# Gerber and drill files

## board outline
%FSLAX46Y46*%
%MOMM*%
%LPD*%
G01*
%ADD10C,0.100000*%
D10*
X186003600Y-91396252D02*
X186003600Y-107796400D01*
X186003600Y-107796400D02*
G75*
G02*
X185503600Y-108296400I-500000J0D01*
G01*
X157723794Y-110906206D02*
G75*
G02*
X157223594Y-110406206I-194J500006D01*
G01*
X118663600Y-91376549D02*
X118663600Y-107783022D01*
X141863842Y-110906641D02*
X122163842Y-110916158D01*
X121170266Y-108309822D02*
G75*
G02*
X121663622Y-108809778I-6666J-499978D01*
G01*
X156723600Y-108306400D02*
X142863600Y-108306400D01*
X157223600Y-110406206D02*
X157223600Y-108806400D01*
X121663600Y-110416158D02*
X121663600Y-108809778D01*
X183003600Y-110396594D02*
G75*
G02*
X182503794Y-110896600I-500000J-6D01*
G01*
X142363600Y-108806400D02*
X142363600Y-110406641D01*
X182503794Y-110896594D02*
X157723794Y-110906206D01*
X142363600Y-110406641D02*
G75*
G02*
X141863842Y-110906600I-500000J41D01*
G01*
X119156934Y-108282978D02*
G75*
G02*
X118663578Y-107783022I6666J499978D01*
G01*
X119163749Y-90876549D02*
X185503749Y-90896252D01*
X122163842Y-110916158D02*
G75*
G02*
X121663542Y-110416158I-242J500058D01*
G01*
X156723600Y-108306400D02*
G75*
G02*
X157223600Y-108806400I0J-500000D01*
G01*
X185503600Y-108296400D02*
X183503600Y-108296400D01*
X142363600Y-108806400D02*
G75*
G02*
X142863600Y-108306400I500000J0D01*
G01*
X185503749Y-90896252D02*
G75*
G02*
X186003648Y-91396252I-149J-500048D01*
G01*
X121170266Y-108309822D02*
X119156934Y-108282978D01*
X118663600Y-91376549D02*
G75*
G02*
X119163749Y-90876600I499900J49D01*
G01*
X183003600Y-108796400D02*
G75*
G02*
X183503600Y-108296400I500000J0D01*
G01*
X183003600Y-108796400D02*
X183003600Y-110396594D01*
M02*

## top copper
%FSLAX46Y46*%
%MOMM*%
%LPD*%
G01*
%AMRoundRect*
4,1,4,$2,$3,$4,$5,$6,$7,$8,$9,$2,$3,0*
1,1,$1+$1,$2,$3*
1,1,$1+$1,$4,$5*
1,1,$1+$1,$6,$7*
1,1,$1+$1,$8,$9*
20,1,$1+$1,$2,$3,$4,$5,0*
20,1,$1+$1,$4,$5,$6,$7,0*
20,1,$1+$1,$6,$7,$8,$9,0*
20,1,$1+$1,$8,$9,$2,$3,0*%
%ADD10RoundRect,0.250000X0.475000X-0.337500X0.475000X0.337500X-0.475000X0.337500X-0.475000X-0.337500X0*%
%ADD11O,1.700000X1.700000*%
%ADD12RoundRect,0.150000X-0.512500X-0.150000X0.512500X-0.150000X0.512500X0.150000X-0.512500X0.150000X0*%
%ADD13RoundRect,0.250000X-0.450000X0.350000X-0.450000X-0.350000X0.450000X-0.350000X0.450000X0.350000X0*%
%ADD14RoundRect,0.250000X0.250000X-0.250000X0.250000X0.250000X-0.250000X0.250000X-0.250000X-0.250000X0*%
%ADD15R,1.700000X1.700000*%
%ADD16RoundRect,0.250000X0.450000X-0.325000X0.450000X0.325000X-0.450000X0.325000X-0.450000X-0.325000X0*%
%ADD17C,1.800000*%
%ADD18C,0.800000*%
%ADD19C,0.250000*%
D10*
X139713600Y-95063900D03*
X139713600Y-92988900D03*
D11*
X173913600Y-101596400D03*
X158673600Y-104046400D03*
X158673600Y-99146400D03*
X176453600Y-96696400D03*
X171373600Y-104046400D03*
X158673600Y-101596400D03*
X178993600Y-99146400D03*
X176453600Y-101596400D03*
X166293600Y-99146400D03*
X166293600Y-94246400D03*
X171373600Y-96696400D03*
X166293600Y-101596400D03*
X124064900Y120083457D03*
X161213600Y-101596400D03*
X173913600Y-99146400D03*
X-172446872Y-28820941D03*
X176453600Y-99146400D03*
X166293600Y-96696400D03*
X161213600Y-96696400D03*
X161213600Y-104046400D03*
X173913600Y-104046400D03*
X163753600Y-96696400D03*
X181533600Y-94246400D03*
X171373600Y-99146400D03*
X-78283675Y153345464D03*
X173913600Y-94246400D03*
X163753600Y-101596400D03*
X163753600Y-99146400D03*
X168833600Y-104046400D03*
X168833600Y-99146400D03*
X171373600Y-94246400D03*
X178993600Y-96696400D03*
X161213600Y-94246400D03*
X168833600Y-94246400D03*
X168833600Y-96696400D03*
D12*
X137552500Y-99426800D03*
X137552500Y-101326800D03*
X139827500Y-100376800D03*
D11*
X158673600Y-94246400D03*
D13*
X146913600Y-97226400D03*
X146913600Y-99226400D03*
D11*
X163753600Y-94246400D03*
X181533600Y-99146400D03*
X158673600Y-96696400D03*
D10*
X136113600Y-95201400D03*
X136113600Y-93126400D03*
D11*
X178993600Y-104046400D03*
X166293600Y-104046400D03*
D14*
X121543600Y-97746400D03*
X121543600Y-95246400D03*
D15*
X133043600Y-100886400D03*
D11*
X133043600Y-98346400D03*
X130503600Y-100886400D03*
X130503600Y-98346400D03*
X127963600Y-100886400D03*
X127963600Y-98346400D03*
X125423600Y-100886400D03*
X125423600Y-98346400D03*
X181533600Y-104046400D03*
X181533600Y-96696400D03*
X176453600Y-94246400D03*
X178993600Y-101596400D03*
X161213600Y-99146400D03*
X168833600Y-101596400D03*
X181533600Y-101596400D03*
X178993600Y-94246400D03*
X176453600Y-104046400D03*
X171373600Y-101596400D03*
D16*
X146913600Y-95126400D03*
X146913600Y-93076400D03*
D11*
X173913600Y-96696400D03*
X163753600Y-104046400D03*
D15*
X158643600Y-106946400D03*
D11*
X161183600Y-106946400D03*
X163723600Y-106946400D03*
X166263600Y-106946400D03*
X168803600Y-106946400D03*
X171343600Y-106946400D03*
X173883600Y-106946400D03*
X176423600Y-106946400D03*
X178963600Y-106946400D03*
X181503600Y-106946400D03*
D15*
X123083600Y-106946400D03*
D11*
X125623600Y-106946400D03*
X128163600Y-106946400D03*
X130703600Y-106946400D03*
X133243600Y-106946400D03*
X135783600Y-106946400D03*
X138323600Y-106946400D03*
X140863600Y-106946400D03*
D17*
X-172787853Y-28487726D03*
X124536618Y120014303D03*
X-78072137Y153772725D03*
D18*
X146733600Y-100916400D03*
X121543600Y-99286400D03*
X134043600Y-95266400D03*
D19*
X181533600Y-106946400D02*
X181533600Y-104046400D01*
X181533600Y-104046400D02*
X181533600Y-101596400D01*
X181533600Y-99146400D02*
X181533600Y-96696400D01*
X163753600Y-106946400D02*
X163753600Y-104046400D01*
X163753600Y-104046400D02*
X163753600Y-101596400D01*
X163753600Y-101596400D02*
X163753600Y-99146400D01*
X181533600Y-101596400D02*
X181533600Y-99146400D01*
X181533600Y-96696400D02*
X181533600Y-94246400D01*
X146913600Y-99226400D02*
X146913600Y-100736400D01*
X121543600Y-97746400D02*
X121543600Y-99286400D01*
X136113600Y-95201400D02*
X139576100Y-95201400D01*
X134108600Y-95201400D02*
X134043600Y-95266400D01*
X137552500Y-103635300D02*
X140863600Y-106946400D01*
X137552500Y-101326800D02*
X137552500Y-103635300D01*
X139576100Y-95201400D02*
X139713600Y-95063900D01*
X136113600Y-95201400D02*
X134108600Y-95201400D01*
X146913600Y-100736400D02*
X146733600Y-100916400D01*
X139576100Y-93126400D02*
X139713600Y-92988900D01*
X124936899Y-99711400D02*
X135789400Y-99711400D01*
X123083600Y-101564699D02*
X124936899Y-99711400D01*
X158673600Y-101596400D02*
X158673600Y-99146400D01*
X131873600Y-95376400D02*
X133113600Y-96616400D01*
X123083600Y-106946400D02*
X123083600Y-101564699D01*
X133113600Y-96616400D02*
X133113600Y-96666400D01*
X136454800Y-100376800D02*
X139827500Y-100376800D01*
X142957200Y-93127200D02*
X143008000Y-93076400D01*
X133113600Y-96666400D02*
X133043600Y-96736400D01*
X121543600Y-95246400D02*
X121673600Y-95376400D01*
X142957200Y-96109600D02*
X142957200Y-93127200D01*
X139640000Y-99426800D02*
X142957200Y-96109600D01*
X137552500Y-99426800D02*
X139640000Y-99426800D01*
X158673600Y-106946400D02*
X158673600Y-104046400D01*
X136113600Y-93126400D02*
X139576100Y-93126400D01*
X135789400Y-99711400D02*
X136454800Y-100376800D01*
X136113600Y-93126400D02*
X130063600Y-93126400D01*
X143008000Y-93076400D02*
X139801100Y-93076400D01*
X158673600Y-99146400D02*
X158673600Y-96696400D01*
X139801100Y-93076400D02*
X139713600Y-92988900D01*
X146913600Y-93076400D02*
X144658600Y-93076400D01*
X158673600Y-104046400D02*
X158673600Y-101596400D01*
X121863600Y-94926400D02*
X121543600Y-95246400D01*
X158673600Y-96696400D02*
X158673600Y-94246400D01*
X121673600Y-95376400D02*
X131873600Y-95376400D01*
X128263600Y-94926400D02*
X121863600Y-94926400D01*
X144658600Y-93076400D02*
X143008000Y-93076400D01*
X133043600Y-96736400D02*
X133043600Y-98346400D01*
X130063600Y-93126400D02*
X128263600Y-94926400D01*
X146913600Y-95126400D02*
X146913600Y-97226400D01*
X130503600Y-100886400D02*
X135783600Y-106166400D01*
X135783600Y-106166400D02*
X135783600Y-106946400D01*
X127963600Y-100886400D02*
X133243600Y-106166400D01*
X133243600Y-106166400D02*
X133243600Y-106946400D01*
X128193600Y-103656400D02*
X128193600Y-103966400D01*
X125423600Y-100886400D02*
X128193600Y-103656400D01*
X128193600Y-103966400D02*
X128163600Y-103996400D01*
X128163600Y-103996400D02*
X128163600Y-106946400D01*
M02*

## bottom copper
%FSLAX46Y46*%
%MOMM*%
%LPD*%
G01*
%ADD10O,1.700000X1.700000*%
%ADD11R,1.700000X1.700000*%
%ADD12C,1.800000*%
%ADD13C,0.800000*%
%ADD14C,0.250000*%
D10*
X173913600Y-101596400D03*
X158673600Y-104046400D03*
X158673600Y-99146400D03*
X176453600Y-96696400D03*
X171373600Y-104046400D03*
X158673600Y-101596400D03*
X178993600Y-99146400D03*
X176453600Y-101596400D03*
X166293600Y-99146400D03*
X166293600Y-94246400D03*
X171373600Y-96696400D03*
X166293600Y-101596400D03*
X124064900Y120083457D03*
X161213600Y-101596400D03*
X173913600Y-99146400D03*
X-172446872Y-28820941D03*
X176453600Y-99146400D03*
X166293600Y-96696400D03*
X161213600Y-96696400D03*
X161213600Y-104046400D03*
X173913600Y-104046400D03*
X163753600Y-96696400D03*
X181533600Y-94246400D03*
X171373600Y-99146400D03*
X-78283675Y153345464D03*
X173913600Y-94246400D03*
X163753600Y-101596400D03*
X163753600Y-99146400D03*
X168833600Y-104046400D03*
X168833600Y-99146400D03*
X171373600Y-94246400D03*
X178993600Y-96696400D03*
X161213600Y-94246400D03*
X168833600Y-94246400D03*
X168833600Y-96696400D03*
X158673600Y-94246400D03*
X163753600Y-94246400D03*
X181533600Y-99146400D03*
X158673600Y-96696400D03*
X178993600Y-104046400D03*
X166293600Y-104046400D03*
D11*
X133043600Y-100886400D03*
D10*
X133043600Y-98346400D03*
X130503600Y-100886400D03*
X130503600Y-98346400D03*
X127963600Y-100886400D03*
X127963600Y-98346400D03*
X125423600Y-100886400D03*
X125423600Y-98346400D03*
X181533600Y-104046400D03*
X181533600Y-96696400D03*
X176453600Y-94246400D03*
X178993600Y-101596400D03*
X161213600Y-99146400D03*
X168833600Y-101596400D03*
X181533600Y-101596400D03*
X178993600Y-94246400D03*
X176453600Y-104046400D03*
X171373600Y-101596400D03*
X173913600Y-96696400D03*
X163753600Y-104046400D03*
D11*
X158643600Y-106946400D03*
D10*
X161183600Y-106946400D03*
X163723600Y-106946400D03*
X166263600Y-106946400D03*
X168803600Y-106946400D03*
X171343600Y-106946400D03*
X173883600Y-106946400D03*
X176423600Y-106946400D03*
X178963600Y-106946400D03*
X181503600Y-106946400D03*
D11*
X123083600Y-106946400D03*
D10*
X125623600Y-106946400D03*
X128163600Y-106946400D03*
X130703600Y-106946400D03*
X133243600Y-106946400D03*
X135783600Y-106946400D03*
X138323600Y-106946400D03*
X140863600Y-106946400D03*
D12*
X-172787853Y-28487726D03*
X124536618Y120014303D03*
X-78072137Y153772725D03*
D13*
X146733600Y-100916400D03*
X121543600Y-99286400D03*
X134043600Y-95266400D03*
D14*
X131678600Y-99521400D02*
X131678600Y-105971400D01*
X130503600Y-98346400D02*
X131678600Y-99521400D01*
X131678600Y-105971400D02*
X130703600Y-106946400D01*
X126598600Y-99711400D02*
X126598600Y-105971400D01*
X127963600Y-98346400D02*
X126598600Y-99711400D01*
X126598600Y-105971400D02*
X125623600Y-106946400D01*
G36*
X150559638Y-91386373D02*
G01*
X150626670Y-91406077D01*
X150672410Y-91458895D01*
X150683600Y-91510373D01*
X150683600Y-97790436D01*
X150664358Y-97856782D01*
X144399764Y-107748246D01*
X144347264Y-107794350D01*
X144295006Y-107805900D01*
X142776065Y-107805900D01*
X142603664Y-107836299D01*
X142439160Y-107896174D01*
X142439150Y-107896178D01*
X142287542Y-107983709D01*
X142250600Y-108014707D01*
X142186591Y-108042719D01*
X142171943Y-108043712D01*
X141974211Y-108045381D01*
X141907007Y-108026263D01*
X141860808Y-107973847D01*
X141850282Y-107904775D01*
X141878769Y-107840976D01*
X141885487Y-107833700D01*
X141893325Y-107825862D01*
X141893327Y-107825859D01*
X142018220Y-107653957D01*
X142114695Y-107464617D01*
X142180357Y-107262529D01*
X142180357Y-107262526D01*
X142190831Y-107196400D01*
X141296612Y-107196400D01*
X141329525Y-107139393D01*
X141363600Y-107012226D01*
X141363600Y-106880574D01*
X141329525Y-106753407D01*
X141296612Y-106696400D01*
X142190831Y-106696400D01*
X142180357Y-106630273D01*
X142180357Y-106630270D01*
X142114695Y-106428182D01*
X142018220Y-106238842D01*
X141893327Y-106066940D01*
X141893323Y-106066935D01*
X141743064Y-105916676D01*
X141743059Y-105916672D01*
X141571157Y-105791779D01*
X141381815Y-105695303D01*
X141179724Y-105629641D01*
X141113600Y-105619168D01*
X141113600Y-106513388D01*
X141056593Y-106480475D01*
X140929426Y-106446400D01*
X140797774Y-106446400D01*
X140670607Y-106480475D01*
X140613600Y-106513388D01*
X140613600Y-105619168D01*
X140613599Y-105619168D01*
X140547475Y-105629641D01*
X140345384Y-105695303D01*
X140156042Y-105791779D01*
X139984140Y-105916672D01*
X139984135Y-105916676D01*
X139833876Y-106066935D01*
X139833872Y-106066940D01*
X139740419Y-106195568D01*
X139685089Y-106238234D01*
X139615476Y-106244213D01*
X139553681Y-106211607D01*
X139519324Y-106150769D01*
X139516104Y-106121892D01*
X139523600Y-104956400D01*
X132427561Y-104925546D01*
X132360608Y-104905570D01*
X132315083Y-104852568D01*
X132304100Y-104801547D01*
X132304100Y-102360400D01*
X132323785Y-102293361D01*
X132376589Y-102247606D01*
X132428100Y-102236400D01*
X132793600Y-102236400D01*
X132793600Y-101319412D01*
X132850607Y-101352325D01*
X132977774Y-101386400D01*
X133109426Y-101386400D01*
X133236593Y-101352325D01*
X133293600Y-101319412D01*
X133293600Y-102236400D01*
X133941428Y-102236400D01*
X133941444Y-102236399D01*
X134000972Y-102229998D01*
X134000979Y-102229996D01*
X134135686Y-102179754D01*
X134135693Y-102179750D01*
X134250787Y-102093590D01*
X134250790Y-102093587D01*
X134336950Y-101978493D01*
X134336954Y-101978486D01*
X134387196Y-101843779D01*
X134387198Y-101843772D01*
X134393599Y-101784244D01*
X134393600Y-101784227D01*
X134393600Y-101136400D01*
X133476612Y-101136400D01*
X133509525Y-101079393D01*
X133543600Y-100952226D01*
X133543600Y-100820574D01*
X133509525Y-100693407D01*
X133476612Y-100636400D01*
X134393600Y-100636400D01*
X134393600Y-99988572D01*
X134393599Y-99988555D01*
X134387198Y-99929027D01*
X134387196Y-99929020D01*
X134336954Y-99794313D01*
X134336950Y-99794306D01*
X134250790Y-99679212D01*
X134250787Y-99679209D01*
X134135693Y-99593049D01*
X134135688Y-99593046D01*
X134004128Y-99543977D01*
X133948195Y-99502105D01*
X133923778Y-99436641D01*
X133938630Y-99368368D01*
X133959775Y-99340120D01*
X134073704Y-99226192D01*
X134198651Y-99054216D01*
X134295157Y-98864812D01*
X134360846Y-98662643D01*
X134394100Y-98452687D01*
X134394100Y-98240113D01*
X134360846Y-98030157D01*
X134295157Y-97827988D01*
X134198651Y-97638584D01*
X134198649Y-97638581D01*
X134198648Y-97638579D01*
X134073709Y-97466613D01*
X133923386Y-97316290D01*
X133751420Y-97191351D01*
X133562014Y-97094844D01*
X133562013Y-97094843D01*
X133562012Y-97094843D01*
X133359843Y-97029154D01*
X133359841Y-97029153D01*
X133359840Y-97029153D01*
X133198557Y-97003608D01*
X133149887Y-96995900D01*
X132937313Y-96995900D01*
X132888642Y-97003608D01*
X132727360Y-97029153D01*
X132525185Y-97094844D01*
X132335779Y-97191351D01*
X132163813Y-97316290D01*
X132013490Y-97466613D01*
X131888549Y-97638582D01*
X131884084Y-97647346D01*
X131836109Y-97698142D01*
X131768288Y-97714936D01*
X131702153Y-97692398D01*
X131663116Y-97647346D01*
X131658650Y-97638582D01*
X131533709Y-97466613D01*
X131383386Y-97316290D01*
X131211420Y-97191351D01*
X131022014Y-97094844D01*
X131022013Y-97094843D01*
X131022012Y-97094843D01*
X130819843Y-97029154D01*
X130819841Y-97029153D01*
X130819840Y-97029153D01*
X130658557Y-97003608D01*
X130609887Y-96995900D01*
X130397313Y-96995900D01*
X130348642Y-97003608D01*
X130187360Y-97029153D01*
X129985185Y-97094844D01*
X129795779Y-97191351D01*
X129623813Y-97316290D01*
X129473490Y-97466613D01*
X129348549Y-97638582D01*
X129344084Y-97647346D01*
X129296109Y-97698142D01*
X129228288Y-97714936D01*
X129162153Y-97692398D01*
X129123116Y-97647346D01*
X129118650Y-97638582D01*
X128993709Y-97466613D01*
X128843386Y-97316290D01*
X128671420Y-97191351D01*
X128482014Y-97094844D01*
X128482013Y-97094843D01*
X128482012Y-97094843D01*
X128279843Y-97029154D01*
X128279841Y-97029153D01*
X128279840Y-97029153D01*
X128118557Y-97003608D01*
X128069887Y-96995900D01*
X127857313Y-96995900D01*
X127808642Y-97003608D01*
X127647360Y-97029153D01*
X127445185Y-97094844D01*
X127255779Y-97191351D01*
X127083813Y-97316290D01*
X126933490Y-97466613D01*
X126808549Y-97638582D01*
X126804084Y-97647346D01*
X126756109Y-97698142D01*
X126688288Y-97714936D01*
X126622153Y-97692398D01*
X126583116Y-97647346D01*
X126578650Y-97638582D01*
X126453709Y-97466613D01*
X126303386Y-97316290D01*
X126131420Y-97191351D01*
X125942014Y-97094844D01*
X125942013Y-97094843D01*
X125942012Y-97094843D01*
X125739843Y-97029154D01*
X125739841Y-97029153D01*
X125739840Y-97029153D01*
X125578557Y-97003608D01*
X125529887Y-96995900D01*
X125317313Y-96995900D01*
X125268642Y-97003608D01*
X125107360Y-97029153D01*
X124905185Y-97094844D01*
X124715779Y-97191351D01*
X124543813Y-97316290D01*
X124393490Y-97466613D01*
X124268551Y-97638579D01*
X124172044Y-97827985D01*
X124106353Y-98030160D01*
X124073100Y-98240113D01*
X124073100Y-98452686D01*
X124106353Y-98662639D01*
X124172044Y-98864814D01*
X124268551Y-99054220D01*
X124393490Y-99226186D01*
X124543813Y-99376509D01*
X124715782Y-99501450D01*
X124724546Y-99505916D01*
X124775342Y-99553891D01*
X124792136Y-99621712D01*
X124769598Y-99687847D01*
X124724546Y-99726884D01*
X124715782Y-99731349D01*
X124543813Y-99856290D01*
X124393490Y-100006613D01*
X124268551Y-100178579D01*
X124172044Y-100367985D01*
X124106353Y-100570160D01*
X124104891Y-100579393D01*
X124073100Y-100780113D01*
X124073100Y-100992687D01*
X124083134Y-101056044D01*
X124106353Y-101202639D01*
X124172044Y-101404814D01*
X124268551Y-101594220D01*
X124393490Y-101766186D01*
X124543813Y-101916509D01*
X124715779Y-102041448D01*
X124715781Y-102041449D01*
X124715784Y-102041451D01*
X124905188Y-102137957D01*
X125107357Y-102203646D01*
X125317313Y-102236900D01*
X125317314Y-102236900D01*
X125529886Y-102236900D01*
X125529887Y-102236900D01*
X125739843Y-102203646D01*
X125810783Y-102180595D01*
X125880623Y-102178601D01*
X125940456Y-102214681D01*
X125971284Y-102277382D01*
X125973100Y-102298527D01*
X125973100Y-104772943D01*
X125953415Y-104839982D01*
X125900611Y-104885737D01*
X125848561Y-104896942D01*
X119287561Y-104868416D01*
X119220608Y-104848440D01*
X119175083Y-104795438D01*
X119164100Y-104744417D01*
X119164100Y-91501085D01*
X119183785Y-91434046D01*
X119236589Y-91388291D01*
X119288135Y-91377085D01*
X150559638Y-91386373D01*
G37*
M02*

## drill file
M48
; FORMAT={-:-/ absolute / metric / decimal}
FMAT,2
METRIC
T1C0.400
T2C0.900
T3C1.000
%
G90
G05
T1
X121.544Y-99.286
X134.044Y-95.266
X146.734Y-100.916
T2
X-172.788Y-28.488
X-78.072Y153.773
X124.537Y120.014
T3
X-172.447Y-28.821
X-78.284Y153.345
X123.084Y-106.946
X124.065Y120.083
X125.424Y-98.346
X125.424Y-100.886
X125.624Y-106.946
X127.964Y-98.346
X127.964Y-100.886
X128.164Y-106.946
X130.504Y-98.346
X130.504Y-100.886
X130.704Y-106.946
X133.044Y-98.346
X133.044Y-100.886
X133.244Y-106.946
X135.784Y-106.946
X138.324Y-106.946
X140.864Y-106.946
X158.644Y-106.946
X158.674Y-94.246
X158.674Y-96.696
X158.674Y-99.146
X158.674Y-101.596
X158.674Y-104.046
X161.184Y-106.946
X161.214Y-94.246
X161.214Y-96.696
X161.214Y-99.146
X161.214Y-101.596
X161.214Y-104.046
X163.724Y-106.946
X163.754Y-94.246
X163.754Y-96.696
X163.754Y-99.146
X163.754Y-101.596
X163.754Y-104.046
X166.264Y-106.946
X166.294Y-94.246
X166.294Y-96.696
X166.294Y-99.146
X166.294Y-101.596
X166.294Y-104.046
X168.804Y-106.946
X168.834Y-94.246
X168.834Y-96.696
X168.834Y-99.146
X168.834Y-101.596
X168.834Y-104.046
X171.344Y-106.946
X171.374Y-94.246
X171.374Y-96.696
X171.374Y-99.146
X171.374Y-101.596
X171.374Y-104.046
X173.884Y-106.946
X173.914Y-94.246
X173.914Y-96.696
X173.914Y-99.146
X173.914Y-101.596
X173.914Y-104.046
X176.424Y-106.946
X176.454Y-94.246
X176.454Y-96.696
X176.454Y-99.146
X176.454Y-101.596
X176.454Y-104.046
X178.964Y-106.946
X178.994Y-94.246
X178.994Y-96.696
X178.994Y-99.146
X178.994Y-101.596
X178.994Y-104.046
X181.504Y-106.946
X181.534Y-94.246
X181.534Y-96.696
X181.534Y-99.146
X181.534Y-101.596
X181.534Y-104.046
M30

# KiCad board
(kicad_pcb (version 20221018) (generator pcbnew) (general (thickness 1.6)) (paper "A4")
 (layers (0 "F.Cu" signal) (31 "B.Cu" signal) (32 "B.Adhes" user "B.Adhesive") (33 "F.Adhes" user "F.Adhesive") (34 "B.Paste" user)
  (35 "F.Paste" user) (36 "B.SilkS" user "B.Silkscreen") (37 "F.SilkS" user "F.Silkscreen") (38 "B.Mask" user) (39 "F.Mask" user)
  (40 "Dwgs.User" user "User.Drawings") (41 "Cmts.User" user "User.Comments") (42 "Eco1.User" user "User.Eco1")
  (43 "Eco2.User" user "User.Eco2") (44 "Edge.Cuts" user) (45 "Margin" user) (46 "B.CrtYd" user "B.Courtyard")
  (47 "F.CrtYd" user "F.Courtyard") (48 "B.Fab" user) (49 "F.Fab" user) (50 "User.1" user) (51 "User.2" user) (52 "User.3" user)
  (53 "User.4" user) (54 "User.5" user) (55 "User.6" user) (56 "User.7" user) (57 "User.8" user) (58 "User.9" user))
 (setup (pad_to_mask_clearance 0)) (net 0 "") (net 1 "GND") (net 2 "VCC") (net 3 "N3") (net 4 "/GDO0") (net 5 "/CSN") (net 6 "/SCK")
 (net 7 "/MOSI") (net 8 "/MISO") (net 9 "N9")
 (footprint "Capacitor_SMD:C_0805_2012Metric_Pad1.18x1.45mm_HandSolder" (layer "F.Cu") (at 139.7136 94.0264 90)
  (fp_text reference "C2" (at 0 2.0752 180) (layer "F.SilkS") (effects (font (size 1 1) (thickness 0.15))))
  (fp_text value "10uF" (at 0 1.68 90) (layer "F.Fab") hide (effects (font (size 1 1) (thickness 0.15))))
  (pad "1" smd roundrect (at -1.0375 0 90) (size 1.175 1.45) (layers "F.Cu" "F.Paste" "F.Mask") (roundrect_rratio 0.2127659574)
   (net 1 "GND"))
  (pad "2" smd roundrect (at 1.0375 0 90) (size 1.175 1.45) (layers "F.Cu" "F.Paste" "F.Mask") (roundrect_rratio 0.2127659574) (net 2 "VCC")))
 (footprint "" (layer "F.Cu") (at 173.9136 101.5964)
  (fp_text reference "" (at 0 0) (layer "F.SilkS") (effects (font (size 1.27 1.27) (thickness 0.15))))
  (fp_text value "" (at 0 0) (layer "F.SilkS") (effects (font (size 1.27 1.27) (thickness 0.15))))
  (pad "" thru_hole oval (at 0 0 270) (size 1.7 1.7) (drill 1) (layers "*.Cu" "*.Mask")))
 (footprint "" (layer "F.Cu") (at 158.6736 104.0464)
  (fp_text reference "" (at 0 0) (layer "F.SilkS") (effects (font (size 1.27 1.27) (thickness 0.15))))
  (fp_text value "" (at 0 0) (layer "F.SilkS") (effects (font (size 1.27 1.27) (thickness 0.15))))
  (pad "" thru_hole oval (at 0 0 270) (size 1.7 1.7) (drill 1) (layers "*.Cu" "*.Mask")))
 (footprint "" (layer "F.Cu") (at 158.6736 99.1464)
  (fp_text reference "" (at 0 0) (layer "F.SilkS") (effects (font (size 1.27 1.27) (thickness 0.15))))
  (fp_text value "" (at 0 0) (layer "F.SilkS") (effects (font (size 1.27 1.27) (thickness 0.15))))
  (pad "" thru_hole oval (at 0 0 270) (size 1.7 1.7) (drill 1) (layers "*.Cu" "*.Mask")))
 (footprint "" (layer "F.Cu") (at 176.4536 96.6964)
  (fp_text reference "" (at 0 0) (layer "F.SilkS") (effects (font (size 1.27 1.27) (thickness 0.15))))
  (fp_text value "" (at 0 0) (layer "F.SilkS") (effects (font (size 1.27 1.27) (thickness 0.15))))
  (pad "" thru_hole oval (at 0 0 270) (size 1.7 1.7) (drill 1) (layers "*.Cu" "*.Mask")))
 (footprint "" (layer "F.Cu") (at 171.3736 104.0464)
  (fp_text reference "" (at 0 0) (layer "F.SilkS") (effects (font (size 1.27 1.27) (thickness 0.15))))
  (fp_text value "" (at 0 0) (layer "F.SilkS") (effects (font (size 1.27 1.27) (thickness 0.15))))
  (pad "" thru_hole oval (at 0 0 270) (size 1.7 1.7) (drill 1) (layers "*.Cu" "*.Mask")))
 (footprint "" (layer "F.Cu") (at 158.6736 101.5964)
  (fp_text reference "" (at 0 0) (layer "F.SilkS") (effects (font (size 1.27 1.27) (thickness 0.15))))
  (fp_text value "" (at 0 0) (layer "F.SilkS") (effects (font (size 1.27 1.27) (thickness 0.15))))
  (pad "" thru_hole oval (at 0 0 270) (size 1.7 1.7) (drill 1) (layers "*.Cu" "*.Mask")))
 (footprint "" (layer "F.Cu") (at 178.9936 99.1464)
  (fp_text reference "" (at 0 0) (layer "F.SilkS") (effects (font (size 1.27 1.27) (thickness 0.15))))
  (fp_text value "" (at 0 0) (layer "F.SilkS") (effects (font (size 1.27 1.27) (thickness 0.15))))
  (pad "" thru_hole oval (at 0 0 270) (size 1.7 1.7) (drill 1) (layers "*.Cu" "*.Mask")))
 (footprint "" (layer "F.Cu") (at 176.4536 101.5964)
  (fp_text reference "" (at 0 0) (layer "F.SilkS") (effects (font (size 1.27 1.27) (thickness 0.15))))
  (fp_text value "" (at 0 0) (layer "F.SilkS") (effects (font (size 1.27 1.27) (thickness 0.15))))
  (pad "" thru_hole oval (at 0 0 270) (size 1.7 1.7) (drill 1) (layers "*.Cu" "*.Mask")))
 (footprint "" (layer "F.Cu") (at 166.2936 99.1464)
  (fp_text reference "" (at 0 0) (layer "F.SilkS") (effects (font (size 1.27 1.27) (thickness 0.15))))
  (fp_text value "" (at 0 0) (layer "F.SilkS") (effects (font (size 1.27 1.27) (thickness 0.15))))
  (pad "" thru_hole oval (at 0 0 270) (size 1.7 1.7) (drill 1) (layers "*.Cu" "*.Mask")))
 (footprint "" (layer "F.Cu") (at 166.2936 94.2464)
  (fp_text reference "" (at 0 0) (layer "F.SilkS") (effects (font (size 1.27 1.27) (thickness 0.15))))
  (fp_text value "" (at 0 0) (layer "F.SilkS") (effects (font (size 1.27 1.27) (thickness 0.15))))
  (pad "" thru_hole oval (at 0 0 270) (size 1.7 1.7) (drill 1) (layers "*.Cu" "*.Mask")))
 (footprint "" (layer "F.Cu") (at 171.3736 96.6964)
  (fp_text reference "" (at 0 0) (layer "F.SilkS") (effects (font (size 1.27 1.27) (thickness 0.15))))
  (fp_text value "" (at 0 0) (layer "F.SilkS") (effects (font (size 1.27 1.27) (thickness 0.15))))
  (pad "" thru_hole oval (at 0 0 270) (size 1.7 1.7) (drill 1) (layers "*.Cu" "*.Mask")))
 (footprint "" (layer "F.Cu") (at 166.2936 101.5964)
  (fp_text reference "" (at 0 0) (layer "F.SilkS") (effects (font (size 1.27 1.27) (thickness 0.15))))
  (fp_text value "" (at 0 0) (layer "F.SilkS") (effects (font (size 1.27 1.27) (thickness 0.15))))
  (pad "" thru_hole oval (at 0 0 270) (size 1.7 1.7) (drill 1) (layers "*.Cu" "*.Mask")))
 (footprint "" (layer "F.Cu") (at 124.0649 -120.083457)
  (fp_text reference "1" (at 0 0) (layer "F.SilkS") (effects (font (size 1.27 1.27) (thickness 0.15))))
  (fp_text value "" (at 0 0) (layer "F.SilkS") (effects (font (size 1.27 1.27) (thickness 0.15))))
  (pad "" thru_hole oval (at 0 0 270) (size 1.7 1.7) (drill 1) (layers "*.Cu" "*.Mask")))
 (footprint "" (layer "F.Cu") (at 161.2136 101.5964)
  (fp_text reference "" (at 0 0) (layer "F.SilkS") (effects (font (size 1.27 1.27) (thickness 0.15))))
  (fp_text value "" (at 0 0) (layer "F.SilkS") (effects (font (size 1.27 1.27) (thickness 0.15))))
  (pad "" thru_hole oval (at 0 0 270) (size 1.7 1.7) (drill 1) (layers "*.Cu" "*.Mask")))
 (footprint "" (layer "F.Cu") (at 173.9136 99.1464)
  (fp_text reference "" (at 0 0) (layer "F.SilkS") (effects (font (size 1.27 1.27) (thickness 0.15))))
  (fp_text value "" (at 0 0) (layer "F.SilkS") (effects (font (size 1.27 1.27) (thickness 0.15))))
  (pad "" thru_hole oval (at 0 0 270) (size 1.7 1.7) (drill 1) (layers "*.Cu" "*.Mask")))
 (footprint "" (layer "F.Cu") (at -172.446872 28.820941)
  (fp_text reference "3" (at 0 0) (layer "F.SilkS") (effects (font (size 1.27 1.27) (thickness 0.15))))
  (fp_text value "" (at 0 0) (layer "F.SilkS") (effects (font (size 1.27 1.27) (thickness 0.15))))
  (pad "" thru_hole oval (at 0 0 270) (size 1.7 1.7) (drill 1) (layers "*.Cu" "*.Mask")))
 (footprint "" (layer "F.Cu") (at 176.4536 99.1464)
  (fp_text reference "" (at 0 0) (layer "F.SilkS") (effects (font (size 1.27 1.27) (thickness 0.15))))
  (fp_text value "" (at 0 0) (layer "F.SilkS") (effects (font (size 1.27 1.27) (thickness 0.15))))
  (pad "" thru_hole oval (at 0 0 270) (size 1.7 1.7) (drill 1) (layers "*.Cu" "*.Mask")))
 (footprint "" (layer "F.Cu") (at 166.2936 96.6964)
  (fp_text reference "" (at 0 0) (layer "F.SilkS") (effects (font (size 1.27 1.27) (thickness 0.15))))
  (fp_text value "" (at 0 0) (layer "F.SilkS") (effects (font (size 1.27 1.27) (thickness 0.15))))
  (pad "" thru_hole oval (at 0 0 270) (size 1.7 1.7) (drill 1) (layers "*.Cu" "*.Mask")))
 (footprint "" (layer "F.Cu") (at 161.2136 96.6964)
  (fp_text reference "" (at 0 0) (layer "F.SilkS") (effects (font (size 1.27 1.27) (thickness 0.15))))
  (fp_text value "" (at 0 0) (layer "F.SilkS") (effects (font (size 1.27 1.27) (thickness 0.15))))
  (pad "" thru_hole oval (at 0 0 270) (size 1.7 1.7) (drill 1) (layers "*.Cu" "*.Mask")))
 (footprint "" (layer "F.Cu") (at 161.2136 104.0464)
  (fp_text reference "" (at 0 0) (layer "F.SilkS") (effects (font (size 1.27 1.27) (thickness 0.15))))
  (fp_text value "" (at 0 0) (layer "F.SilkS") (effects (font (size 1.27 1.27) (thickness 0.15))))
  (pad "" thru_hole oval (at 0 0 270) (size 1.7 1.7) (drill 1) (layers "*.Cu" "*.Mask")))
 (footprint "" (layer "F.Cu") (at 173.9136 104.0464)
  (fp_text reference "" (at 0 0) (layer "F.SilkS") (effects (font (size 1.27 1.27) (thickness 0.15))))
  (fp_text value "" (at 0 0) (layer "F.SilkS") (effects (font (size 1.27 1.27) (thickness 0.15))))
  (pad "" thru_hole oval (at 0 0 270) (size 1.7 1.7) (drill 1) (layers "*.Cu" "*.Mask")))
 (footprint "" (layer "F.Cu") (at 163.7536 96.6964)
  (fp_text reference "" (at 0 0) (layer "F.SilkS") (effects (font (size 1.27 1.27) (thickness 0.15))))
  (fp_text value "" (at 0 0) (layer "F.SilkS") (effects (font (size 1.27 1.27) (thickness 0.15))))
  (pad "" thru_hole oval (at 0 0 270) (size 1.7 1.7) (drill 1) (layers "*.Cu" "*.Mask")))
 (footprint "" (layer "F.Cu") (at 181.5336 94.2464)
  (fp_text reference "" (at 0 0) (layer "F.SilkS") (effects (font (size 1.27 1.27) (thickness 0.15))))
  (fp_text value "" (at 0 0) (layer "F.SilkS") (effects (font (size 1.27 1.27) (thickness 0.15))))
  (pad "" thru_hole oval (at 0 0 270) (size 1.7 1.7) (drill 1) (layers "*.Cu" "*.Mask")))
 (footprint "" (layer "F.Cu") (at 171.3736 99.1464)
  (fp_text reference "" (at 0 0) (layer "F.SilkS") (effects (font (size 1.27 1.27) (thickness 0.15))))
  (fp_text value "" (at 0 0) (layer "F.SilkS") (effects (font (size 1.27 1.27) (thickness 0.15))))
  (pad "" thru_hole oval (at 0 0 270) (size 1.7 1.7) (drill 1) (layers "*.Cu" "*.Mask")))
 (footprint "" (layer "F.Cu") (at -78.283675 -153.345464)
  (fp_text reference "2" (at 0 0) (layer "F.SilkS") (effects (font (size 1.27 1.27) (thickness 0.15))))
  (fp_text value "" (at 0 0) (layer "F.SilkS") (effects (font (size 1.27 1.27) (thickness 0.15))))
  (pad "" thru_hole oval (at 0 0 270) (size 1.7 1.7) (drill 1) (layers "*.Cu" "*.Mask")))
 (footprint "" (layer "F.Cu") (at 173.9136 94.2464)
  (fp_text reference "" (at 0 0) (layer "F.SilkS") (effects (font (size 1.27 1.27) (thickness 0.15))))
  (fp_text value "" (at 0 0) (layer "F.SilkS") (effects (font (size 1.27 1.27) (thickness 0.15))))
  (pad "" thru_hole oval (at 0 0 270) (size 1.7 1.7) (drill 1) (layers "*.Cu" "*.Mask")))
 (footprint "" (layer "F.Cu") (at 163.7536 101.5964)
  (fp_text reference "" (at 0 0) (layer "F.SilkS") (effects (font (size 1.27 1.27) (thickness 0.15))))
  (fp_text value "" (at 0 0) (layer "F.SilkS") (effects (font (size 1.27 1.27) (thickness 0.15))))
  (pad "" thru_hole oval (at 0 0 270) (size 1.7 1.7) (drill 1) (layers "*.Cu" "*.Mask")))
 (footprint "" (layer "F.Cu") (at 163.7536 99.1464)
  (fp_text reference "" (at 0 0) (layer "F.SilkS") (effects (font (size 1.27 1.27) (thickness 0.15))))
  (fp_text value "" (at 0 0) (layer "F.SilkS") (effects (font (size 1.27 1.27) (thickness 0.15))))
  (pad "" thru_hole oval (at 0 0 270) (size 1.7 1.7) (drill 1) (layers "*.Cu" "*.Mask")))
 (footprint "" (layer "F.Cu") (at 168.8336 104.0464)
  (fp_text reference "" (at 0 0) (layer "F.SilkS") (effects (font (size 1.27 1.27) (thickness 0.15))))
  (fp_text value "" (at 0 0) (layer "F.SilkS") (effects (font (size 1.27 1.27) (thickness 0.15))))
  (pad "" thru_hole oval (at 0 0 270) (size 1.7 1.7) (drill 1) (layers "*.Cu" "*.Mask")))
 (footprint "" (layer "F.Cu") (at 168.8336 99.1464)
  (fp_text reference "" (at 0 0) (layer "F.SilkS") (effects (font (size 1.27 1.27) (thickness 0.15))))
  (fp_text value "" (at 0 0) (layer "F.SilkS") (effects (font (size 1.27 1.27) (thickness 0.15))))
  (pad "" thru_hole oval (at 0 0 270) (size 1.7 1.7) (drill 1) (layers "*.Cu" "*.Mask")))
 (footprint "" (layer "F.Cu") (at 171.3736 94.2464)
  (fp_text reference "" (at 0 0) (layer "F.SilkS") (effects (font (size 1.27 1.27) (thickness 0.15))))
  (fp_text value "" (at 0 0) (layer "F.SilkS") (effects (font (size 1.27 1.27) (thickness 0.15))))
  (pad "" thru_hole oval (at 0 0 270) (size 1.7 1.7) (drill 1) (layers "*.Cu" "*.Mask")))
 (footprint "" (layer "F.Cu") (at 178.9936 96.6964)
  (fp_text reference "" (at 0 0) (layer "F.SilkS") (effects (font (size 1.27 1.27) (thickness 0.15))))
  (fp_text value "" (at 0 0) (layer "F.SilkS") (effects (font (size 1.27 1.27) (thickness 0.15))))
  (pad "" thru_hole oval (at 0 0 270) (size 1.7 1.7) (drill 1) (layers "*.Cu" "*.Mask")))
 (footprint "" (layer "F.Cu") (at 161.2136 94.2464)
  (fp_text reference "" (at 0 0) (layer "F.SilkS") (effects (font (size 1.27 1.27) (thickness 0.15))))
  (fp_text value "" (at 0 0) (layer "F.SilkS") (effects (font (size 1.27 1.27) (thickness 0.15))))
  (pad "" thru_hole oval (at 0 0 270) (size 1.7 1.7) (drill 1) (layers "*.Cu" "*.Mask")))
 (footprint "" (layer "F.Cu") (at 168.8336 94.2464)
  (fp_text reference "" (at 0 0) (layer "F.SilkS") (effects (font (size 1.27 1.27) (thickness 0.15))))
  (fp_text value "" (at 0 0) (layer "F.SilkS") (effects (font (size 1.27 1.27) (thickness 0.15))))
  (pad "" thru_hole oval (at 0 0 270) (size 1.7 1.7) (drill 1) (layers "*.Cu" "*.Mask")))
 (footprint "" (layer "F.Cu") (at 168.8336 96.6964)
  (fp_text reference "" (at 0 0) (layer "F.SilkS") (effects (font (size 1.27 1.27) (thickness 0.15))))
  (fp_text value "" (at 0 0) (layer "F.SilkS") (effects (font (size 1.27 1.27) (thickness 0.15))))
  (pad "" thru_hole oval (at 0 0 270) (size 1.7 1.7) (drill 1) (layers "*.Cu" "*.Mask")))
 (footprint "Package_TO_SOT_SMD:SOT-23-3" (layer "F.Cu") (at 138.69 100.3768)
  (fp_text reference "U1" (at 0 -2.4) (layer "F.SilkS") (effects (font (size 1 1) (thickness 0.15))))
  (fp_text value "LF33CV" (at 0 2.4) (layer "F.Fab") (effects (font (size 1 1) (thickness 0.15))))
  (pad "1" smd roundrect (at -1.1375 -0.95) (size 1.325 0.6) (layers "F.Cu" "F.Paste" "F.Mask") (roundrect_rratio 0.25) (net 2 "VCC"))
  (pad "2" smd roundrect (at -1.1375 0.95) (size 1.325 0.6) (layers "F.Cu" "F.Paste" "F.Mask") (roundrect_rratio 0.25) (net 1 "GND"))
  (pad "3" smd roundrect (at 1.1375 0) (size 1.325 0.6) (layers "F.Cu" "F.Paste" "F.Mask") (roundrect_rratio 0.25) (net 2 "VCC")))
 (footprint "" (layer "F.Cu") (at 158.6736 94.2464)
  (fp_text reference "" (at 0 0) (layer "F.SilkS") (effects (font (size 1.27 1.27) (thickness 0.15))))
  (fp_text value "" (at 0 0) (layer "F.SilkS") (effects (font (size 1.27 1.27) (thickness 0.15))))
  (pad "" thru_hole oval (at 0 0 270) (size 1.7 1.7) (drill 1) (layers "*.Cu" "*.Mask")))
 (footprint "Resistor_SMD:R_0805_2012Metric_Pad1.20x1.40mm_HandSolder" (layer "F.Cu") (at 146.9136 98.2264 -90)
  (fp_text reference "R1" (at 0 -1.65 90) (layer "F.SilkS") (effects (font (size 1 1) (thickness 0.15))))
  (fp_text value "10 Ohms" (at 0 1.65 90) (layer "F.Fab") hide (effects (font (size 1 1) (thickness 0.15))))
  (pad "1" smd roundrect (at -1 0 270) (size 1.2 1.4) (layers "F.Cu" "F.Paste" "F.Mask") (roundrect_rratio 0.2083333333) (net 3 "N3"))
  (pad "2" smd roundrect (at 1 0 270) (size 1.2 1.4) (layers "F.Cu" "F.Paste" "F.Mask") (roundrect_rratio 0.2083333333) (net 1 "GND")))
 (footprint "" (layer "F.Cu") (at 163.7536 94.2464)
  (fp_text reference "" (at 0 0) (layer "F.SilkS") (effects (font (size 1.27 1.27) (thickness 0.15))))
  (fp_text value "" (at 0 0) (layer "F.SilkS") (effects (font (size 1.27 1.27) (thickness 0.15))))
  (pad "" thru_hole oval (at 0 0 270) (size 1.7 1.7) (drill 1) (layers "*.Cu" "*.Mask")))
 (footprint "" (layer "F.Cu") (at 181.5336 99.1464)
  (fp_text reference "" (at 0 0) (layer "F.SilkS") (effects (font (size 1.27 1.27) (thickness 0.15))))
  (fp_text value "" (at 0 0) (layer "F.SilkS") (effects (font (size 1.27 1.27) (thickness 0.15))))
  (pad "" thru_hole oval (at 0 0 270) (size 1.7 1.7) (drill 1) (layers "*.Cu" "*.Mask")))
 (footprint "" (layer "F.Cu") (at 158.6736 96.6964)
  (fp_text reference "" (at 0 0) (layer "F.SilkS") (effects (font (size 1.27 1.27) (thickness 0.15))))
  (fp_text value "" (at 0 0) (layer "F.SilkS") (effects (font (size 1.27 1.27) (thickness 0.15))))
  (pad "" thru_hole oval (at 0 0 270) (size 1.7 1.7) (drill 1) (layers "*.Cu" "*.Mask")))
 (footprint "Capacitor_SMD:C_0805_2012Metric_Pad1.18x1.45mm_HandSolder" (layer "F.Cu") (at 136.1136 94.1639 90)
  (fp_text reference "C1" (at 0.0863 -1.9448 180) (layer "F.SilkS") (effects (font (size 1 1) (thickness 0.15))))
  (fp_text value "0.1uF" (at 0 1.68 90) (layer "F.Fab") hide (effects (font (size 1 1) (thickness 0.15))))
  (pad "1" smd roundrect (at -1.0375 0 90) (size 1.175 1.45) (layers "F.Cu" "F.Paste" "F.Mask") (roundrect_rratio 0.2127659574)
   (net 1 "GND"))
  (pad "2" smd roundrect (at 1.0375 0 90) (size 1.175 1.45) (layers "F.Cu" "F.Paste" "F.Mask") (roundrect_rratio 0.2127659574) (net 2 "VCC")))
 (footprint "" (layer "F.Cu") (at 178.9936 104.0464)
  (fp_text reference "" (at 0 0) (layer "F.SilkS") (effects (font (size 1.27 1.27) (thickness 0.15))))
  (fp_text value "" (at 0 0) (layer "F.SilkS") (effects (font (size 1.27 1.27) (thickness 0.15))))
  (pad "" thru_hole oval (at 0 0 270) (size 1.7 1.7) (drill 1) (layers "*.Cu" "*.Mask")))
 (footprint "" (layer "F.Cu") (at 166.2936 104.0464)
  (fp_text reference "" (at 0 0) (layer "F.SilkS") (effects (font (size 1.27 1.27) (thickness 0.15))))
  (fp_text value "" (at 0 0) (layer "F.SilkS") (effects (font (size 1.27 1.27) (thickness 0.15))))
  (pad "" thru_hole oval (at 0 0 270) (size 1.7 1.7) (drill 1) (layers "*.Cu" "*.Mask")))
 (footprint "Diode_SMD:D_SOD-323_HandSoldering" (layer "F.Cu") (at 121.5436 96.4964 90)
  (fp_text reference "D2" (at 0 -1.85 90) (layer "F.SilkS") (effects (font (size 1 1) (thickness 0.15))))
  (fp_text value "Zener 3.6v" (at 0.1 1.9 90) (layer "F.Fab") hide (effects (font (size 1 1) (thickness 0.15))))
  (pad "1" smd roundrect (at -1.25 0 90) (size 1 1) (layers "F.Cu" "F.Paste" "F.Mask") (roundrect_rratio 0.25) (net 1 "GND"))
  (pad "2" smd roundrect (at 1.25 0 90) (size 1 1) (layers "F.Cu" "F.Paste" "F.Mask") (roundrect_rratio 0.25) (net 2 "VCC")))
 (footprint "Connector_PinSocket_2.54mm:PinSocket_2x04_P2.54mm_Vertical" (layer "F.Cu") (at 133.0436 100.8864 -90)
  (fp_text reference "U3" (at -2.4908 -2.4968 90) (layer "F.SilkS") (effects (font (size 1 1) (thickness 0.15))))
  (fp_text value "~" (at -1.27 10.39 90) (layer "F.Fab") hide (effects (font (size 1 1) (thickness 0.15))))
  (pad "1" thru_hole rect (at 0 0 270) (size 1.7 1.7) (drill 1) (layers "*.Cu" "*.Mask") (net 1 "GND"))
  (pad "2" thru_hole oval (at -2.54 0 270) (size 1.7 1.7) (drill 1) (layers "*.Cu" "*.Mask") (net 2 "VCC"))
  (pad "3" thru_hole oval (at 0 2.54 270) (size 1.7 1.7) (drill 1) (layers "*.Cu" "*.Mask") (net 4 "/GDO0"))
  (pad "4" thru_hole oval (at -2.54 2.54 270) (size 1.7 1.7) (drill 1) (layers "*.Cu" "*.Mask") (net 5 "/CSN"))
  (pad "5" thru_hole oval (at 0 5.08 270) (size 1.7 1.7) (drill 1) (layers "*.Cu" "*.Mask") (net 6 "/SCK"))
  (pad "6" thru_hole oval (at -2.54 5.08 270) (size 1.7 1.7) (drill 1) (layers "*.Cu" "*.Mask") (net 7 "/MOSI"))
  (pad "7" thru_hole oval (at 0 7.62 270) (size 1.7 1.7) (drill 1) (layers "*.Cu" "*.Mask") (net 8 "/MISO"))
  (pad "8" thru_hole oval (at -2.54 7.62 270) (size 1.7 1.7) (drill 1) (layers "*.Cu" "*.Mask") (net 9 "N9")))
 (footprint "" (layer "F.Cu") (at 181.5336 104.0464)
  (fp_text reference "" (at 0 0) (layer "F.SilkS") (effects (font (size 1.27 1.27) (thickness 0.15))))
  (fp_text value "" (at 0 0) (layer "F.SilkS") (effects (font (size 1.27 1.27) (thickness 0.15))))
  (pad "" thru_hole oval (at 0 0 270) (size 1.7 1.7) (drill 1) (layers "*.Cu" "*.Mask")))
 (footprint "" (layer "F.Cu") (at 181.5336 96.6964)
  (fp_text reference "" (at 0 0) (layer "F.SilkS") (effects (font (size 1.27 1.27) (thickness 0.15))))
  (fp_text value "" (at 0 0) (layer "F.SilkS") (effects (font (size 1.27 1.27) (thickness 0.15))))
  (pad "" thru_hole oval (at 0 0 270) (size 1.7 1.7) (drill 1) (layers "*.Cu" "*.Mask")))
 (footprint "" (layer "F.Cu") (at 176.4536 94.2464)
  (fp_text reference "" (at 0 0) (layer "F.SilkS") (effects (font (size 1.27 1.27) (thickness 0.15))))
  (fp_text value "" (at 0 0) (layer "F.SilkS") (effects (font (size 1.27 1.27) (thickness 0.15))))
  (pad "" thru_hole oval (at 0 0 270) (size 1.7 1.7) (drill 1) (layers "*.Cu" "*.Mask")))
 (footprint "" (layer "F.Cu") (at 178.9936 101.5964)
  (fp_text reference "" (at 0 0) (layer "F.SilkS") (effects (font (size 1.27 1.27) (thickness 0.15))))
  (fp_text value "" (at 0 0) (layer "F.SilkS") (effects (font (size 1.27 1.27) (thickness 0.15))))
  (pad "" thru_hole oval (at 0 0 270) (size 1.7 1.7) (drill 1) (layers "*.Cu" "*.Mask")))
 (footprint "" (layer "F.Cu") (at 161.2136 99.1464)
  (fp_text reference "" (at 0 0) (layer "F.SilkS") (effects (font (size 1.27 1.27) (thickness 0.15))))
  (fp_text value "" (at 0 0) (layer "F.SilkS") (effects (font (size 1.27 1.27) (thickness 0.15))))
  (pad "" thru_hole oval (at 0 0 270) (size 1.7 1.7) (drill 1) (layers "*.Cu" "*.Mask")))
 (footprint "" (layer "F.Cu") (at 168.8336 101.5964)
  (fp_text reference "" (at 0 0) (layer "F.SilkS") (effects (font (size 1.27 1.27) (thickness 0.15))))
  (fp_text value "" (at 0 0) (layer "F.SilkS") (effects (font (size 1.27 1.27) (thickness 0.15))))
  (pad "" thru_hole oval (at 0 0 270) (size 1.7 1.7) (drill 1) (layers "*.Cu" "*.Mask")))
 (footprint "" (layer "F.Cu") (at 181.5336 101.5964)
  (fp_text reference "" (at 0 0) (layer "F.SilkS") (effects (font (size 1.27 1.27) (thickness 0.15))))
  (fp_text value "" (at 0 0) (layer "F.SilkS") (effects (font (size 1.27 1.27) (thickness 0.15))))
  (pad "" thru_hole oval (at 0 0 270) (size 1.7 1.7) (drill 1) (layers "*.Cu" "*.Mask")))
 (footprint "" (layer "F.Cu") (at 178.9936 94.2464)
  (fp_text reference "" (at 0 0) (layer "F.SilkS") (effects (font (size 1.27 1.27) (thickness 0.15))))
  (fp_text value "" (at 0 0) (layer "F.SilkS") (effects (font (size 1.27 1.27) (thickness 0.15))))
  (pad "" thru_hole oval (at 0 0 270) (size 1.7 1.7) (drill 1) (layers "*.Cu" "*.Mask")))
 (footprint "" (layer "F.Cu") (at 176.4536 104.0464)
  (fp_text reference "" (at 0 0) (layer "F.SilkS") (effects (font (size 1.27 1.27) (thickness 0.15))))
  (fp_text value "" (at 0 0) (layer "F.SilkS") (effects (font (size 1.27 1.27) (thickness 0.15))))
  (pad "" thru_hole oval (at 0 0 270) (size 1.7 1.7) (drill 1) (layers "*.Cu" "*.Mask")))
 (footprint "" (layer "F.Cu") (at 171.3736 101.5964)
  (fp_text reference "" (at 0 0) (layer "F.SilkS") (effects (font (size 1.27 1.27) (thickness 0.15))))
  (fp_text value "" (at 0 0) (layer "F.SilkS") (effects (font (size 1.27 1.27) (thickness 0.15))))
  (pad "" thru_hole oval (at 0 0 270) (size 1.7 1.7) (drill 1) (layers "*.Cu" "*.Mask")))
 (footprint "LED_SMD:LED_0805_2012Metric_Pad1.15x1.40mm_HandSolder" (layer "F.Cu") (at 146.9136 94.1014 90)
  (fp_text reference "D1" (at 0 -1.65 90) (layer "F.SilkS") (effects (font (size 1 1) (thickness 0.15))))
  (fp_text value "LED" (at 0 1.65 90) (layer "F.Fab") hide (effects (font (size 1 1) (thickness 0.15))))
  (pad "1" smd roundrect (at -1.025 0 90) (size 1.15 1.4) (layers "F.Cu" "F.Paste" "F.Mask") (roundrect_rratio 0.2173913043) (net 3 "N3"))
  (pad "2" smd roundrect (at 1.025 0 90) (size 1.15 1.4) (layers "F.Cu" "F.Paste" "F.Mask") (roundrect_rratio 0.2173913043) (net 2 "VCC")))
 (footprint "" (layer "F.Cu") (at 173.9136 96.6964)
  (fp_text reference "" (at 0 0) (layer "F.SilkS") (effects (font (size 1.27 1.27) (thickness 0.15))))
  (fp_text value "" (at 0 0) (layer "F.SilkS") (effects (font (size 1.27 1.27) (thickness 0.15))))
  (pad "" thru_hole oval (at 0 0 270) (size 1.7 1.7) (drill 1) (layers "*.Cu" "*.Mask")))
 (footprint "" (layer "F.Cu") (at 163.7536 104.0464)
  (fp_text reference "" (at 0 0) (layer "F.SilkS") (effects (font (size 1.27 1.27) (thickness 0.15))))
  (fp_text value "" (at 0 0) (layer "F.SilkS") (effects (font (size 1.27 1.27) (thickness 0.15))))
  (pad "" thru_hole oval (at 0 0 270) (size 1.7 1.7) (drill 1) (layers "*.Cu" "*.Mask")))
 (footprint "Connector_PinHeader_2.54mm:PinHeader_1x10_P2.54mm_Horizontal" (layer "B.Cu") (at 158.6436 106.9464 -90)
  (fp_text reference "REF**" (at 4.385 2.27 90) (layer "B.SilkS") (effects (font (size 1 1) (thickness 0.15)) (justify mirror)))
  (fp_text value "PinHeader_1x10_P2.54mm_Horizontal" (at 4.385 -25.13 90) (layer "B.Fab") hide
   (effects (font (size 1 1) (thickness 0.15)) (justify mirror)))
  (pad "1" thru_hole rect (at 0 0 270) (size 1.7 1.7) (drill 1) (layers "*.Cu" "*.Mask"))
  (pad "2" thru_hole oval (at 0 -2.54 270) (size 1.7 1.7) (drill 1) (layers "*.Cu" "*.Mask"))
  (pad "3" thru_hole oval (at 0 -5.08 270) (size 1.7 1.7) (drill 1) (layers "*.Cu" "*.Mask"))
  (pad "4" thru_hole oval (at 0 -7.62 270) (size 1.7 1.7) (drill 1) (layers "*.Cu" "*.Mask"))
  (pad "5" thru_hole oval (at 0 -10.16 270) (size 1.7 1.7) (drill 1) (layers "*.Cu" "*.Mask"))
  (pad "6" thru_hole oval (at 0 -12.7 270) (size 1.7 1.7) (drill 1) (layers "*.Cu" "*.Mask"))
  (pad "7" thru_hole oval (at 0 -15.24 270) (size 1.7 1.7) (drill 1) (layers "*.Cu" "*.Mask"))
  (pad "8" thru_hole oval (at 0 -17.78 270) (size 1.7 1.7) (drill 1) (layers "*.Cu" "*.Mask"))
  (pad "9" thru_hole oval (at 0 -20.32 270) (size 1.7 1.7) (drill 1) (layers "*.Cu" "*.Mask"))
  (pad "10" thru_hole oval (at 0 -22.86 270) (size 1.7 1.7) (drill 1) (layers "*.Cu" "*.Mask")))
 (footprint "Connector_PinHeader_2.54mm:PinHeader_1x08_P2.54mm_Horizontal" (layer "B.Cu") (at 123.0836 106.9464 -90)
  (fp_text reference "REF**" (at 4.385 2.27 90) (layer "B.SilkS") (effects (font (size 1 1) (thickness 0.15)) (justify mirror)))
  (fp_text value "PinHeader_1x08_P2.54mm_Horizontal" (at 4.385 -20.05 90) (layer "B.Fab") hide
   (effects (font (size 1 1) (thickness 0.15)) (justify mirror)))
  (pad "1" thru_hole rect (at 0 0 270) (size 1.7 1.7) (drill 1) (layers "*.Cu" "*.Mask") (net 2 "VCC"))
  (pad "2" thru_hole oval (at 0 -2.54 270) (size 1.7 1.7) (drill 1) (layers "*.Cu" "*.Mask") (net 7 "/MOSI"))
  (pad "3" thru_hole oval (at 0 -5.08 270) (size 1.7 1.7) (drill 1) (layers "*.Cu" "*.Mask") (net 8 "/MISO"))
  (pad "4" thru_hole oval (at 0 -7.62 270) (size 1.7 1.7) (drill 1) (layers "*.Cu" "*.Mask") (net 5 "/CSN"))
  (pad "5" thru_hole oval (at 0 -10.16 270) (size 1.7 1.7) (drill 1) (layers "*.Cu" "*.Mask") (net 6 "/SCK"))
  (pad "6" thru_hole oval (at 0 -12.7 270) (size 1.7 1.7) (drill 1) (layers "*.Cu" "*.Mask") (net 4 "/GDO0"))
  (pad "7" thru_hole oval (at 0 -15.24 270) (size 1.7 1.7) (drill 1) (layers "*.Cu" "*.Mask"))
  (pad "8" thru_hole oval (at 0 -17.78 270) (size 1.7 1.7) (drill 1) (layers "*.Cu" "*.Mask") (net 1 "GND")))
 (gr_line (start 186.0036 91.396252) (end 186.0036 107.7964) (stroke (width 0.1) (type default)) (layer "Edge.Cuts"))
 (gr_arc (start 186.0036 107.7964) (mid 185.857153 108.149953) (end 185.5036 108.2964) (stroke (width 0.1) (type default))
  (layer "Edge.Cuts"))
 (gr_arc (start 157.723794 110.906206) (mid 157.370113 110.759828) (end 157.2236 110.406206) (stroke (width 0.1) (type default))
  (layer "Edge.Cuts"))
 (gr_line (start 118.6636 91.376549) (end 118.6636 107.783022) (stroke (width 0.1) (type default)) (layer "Edge.Cuts"))
 (gr_line (start 141.863842 110.906641) (end 122.163842 110.916158) (stroke (width 0.1) (type default)) (layer "Edge.Cuts"))
 (gr_arc (start 121.170266 108.309822) (mid 121.519511 108.458588) (end 121.6636 108.809778) (stroke (width 0.1) (type default))
  (layer "Edge.Cuts"))
 (gr_line (start 156.7236 108.3064) (end 142.8636 108.3064) (stroke (width 0.1) (type default)) (layer "Edge.Cuts"))
 (gr_line (start 157.2236 110.406206) (end 157.2236 108.8064) (stroke (width 0.1) (type default)) (layer "Edge.Cuts"))
 (gr_line (start 121.6636 110.416158) (end 121.6636 108.809778) (stroke (width 0.1) (type default)) (layer "Edge.Cuts"))
 (gr_arc (start 183.0036 110.396594) (mid 182.857224 110.750083) (end 182.503794 110.896594) (stroke (width 0.1) (type default))
  (layer "Edge.Cuts"))
 (gr_line (start 142.3636 108.8064) (end 142.3636 110.406641) (stroke (width 0.1) (type default)) (layer "Edge.Cuts"))
 (gr_line (start 182.503794 110.896594) (end 157.723794 110.906206) (stroke (width 0.1) (type default)) (layer "Edge.Cuts"))
 (gr_arc (start 142.3636 110.406641) (mid 142.217231 110.760118) (end 141.863842 110.906641) (stroke (width 0.1) (type default))
  (layer "Edge.Cuts"))
 (gr_arc (start 119.156934 108.282978) (mid 118.807689 108.134212) (end 118.6636 107.783022) (stroke (width 0.1) (type default))
  (layer "Edge.Cuts"))
 (gr_line (start 119.163749 90.876549) (end 185.503749 90.896252) (stroke (width 0.1) (type default)) (layer "Edge.Cuts"))
 (gr_arc (start 122.163842 110.916158) (mid 121.810147 110.769794) (end 121.6636 110.416158) (stroke (width 0.1) (type default))
  (layer "Edge.Cuts"))
 (gr_arc (start 156.7236 108.3064) (mid 157.077153 108.452847) (end 157.2236 108.8064) (stroke (width 0.1) (type default))
  (layer "Edge.Cuts"))
 (gr_line (start 185.5036 108.2964) (end 183.5036 108.2964) (stroke (width 0.1) (type default)) (layer "Edge.Cuts"))
 (gr_arc (start 142.3636 108.8064) (mid 142.510047 108.452847) (end 142.8636 108.3064) (stroke (width 0.1) (type default))
  (layer "Edge.Cuts"))
 (gr_arc (start 185.503749 90.896252) (mid 185.857188 91.042754) (end 186.0036 91.396252) (stroke (width 0.1) (type default))
  (layer "Edge.Cuts"))
 (gr_line (start 121.170266 108.309822) (end 119.156934 108.282978) (stroke (width 0.1) (type default)) (layer "Edge.Cuts"))
 (gr_arc (start 118.6636 91.376549) (mid 118.810082 91.022911) (end 119.163749 90.876549) (stroke (width 0.1) (type default))
  (layer "Edge.Cuts"))
 (gr_arc (start 183.0036 108.7964) (mid 183.150047 108.442847) (end 183.5036 108.2964) (stroke (width 0.1) (type default))
  (layer "Edge.Cuts"))
 (gr_line (start 183.0036 108.7964) (end 183.0036 110.396594) (stroke (width 0.1) (type default)) (layer "Edge.Cuts"))
 (segment (start 181.5336 106.9464) (end 181.5336 104.0464) (width 0.25) (layer "F.Cu") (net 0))
 (segment (start 181.5336 104.0464) (end 181.5336 101.5964) (width 0.25) (layer "F.Cu") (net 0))
 (segment (start 181.5336 99.1464) (end 181.5336 96.6964) (width 0.25) (layer "F.Cu") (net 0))
 (segment (start 163.7536 106.9464) (end 163.7536 104.0464) (width 0.25) (layer "F.Cu") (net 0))
 (segment (start 163.7536 104.0464) (end 163.7536 101.5964) (width 0.25) (layer "F.Cu") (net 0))
 (segment (start 163.7536 101.5964) (end 163.7536 99.1464) (width 0.25) (layer "F.Cu") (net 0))
 (segment (start 181.5336 101.5964) (end 181.5336 99.1464) (width 0.25) (layer "F.Cu") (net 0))
 (segment (start 181.5336 96.6964) (end 181.5336 94.2464) (width 0.25) (layer "F.Cu") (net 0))
 (via (at -172.787853 28.487726) (size 1.8) (drill 0.9) (layers "F.Cu" "B.Cu") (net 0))
 (via (at 124.536618 -120.014303) (size 1.8) (drill 0.9) (layers "F.Cu" "B.Cu") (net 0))
 (via (at -78.072137 -153.772725) (size 1.8) (drill 0.9) (layers "F.Cu" "B.Cu") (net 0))
 (segment (start 146.9136 99.2264) (end 146.9136 100.7364) (width 0.25) (layer "F.Cu") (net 1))
 (segment (start 121.5436 97.7464) (end 121.5436 99.2864) (width 0.25) (layer "F.Cu") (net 1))
 (segment (start 136.1136 95.2014) (end 139.5761 95.2014) (width 0.25) (layer "F.Cu") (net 1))
 (segment (start 134.1086 95.2014) (end 134.0436 95.2664) (width 0.25) (layer "F.Cu") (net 1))
 (segment (start 137.5525 103.6353) (end 140.8636 106.9464) (width 0.25) (layer "F.Cu") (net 1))
 (segment (start 137.5525 101.3268) (end 137.5525 103.6353) (width 0.25) (layer "F.Cu") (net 1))
 (segment (start 139.5761 95.2014) (end 139.7136 95.0639) (width 0.25) (layer "F.Cu") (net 1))
 (segment (start 136.1136 95.2014) (end 134.1086 95.2014) (width 0.25) (layer "F.Cu") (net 1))
 (segment (start 146.9136 100.7364) (end 146.7336 100.9164) (width 0.25) (layer "F.Cu") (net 1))
 (via (at 146.7336 100.9164) (size 0.8) (drill 0.4) (layers "F.Cu" "B.Cu") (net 1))
 (via (at 121.5436 99.2864) (size 0.8) (drill 0.4) (layers "F.Cu" "B.Cu") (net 1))
 (via (at 134.0436 95.2664) (size 0.8) (drill 0.4) (layers "F.Cu" "B.Cu") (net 1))
 (segment (start 139.5761 93.1264) (end 139.7136 92.9889) (width 0.25) (layer "F.Cu") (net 2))
 (segment (start 124.936899 99.7114) (end 135.7894 99.7114) (width 0.25) (layer "F.Cu") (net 2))
 (segment (start 123.0836 101.564699) (end 124.936899 99.7114) (width 0.25) (layer "F.Cu") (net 2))
 (segment (start 158.6736 101.5964) (end 158.6736 99.1464) (width 0.25) (layer "F.Cu") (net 2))
 (segment (start 131.8736 95.3764) (end 133.1136 96.6164) (width 0.25) (layer "F.Cu") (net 2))
 (segment (start 123.0836 106.9464) (end 123.0836 101.564699) (width 0.25) (layer "F.Cu") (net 2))
 (segment (start 133.1136 96.6164) (end 133.1136 96.6664) (width 0.25) (layer "F.Cu") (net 2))
 (segment (start 136.4548 100.3768) (end 139.8275 100.3768) (width 0.25) (layer "F.Cu") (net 2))
 (segment (start 142.9572 93.1272) (end 143.008 93.0764) (width 0.25) (layer "F.Cu") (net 2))
 (segment (start 133.1136 96.6664) (end 133.0436 96.7364) (width 0.25) (layer "F.Cu") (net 2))
 (segment (start 121.5436 95.2464) (end 121.6736 95.3764) (width 0.25) (layer "F.Cu") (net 2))
 (segment (start 142.9572 96.1096) (end 142.9572 93.1272) (width 0.25) (layer "F.Cu") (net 2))
 (segment (start 139.64 99.4268) (end 142.9572 96.1096) (width 0.25) (layer "F.Cu") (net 2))
 (segment (start 137.5525 99.4268) (end 139.64 99.4268) (width 0.25) (layer "F.Cu") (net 2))
 (segment (start 158.6736 106.9464) (end 158.6736 104.0464) (width 0.25) (layer "F.Cu") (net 2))
 (segment (start 136.1136 93.1264) (end 139.5761 93.1264) (width 0.25) (layer "F.Cu") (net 2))
 (segment (start 135.7894 99.7114) (end 136.4548 100.3768) (width 0.25) (layer "F.Cu") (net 2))
 (segment (start 136.1136 93.1264) (end 130.0636 93.1264) (width 0.25) (layer "F.Cu") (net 2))
 (segment (start 143.008 93.0764) (end 139.8011 93.0764) (width 0.25) (layer "F.Cu") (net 2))
 (segment (start 158.6736 99.1464) (end 158.6736 96.6964) (width 0.25) (layer "F.Cu") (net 2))
 (segment (start 139.8011 93.0764) (end 139.7136 92.9889) (width 0.25) (layer "F.Cu") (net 2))
 (segment (start 146.9136 93.0764) (end 144.6586 93.0764) (width 0.25) (layer "F.Cu") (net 2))
 (segment (start 158.6736 104.0464) (end 158.6736 101.5964) (width 0.25) (layer "F.Cu") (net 2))
 (segment (start 121.8636 94.9264) (end 121.5436 95.2464) (width 0.25) (layer "F.Cu") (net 2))
 (segment (start 158.6736 96.6964) (end 158.6736 94.2464) (width 0.25) (layer "F.Cu") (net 2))
 (segment (start 121.6736 95.3764) (end 131.8736 95.3764) (width 0.25) (layer "F.Cu") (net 2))
 (segment (start 128.2636 94.9264) (end 121.8636 94.9264) (width 0.25) (layer "F.Cu") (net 2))
 (segment (start 144.6586 93.0764) (end 143.008 93.0764) (width 0.25) (layer "F.Cu") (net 2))
 (segment (start 133.0436 96.7364) (end 133.0436 98.3464) (width 0.25) (layer "F.Cu") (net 2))
 (segment (start 130.0636 93.1264) (end 128.2636 94.9264) (width 0.25) (layer "F.Cu") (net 2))
 (segment (start 146.9136 95.1264) (end 146.9136 97.2264) (width 0.25) (layer "F.Cu") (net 3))
 (segment (start 130.5036 100.8864) (end 135.7836 106.1664) (width 0.25) (layer "F.Cu") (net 4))
 (segment (start 135.7836 106.1664) (end 135.7836 106.9464) (width 0.25) (layer "F.Cu") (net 4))
 (segment (start 131.6786 99.5214) (end 131.6786 105.9714) (width 0.25) (layer "B.Cu") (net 5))
 (segment (start 130.5036 98.3464) (end 131.6786 99.5214) (width 0.25) (layer "B.Cu") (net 5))
 (segment (start 131.6786 105.9714) (end 130.7036 106.9464) (width 0.25) (layer "B.Cu") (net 5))
 (segment (start 127.9636 100.8864) (end 133.2436 106.1664) (width 0.25) (layer "F.Cu") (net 6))
 (segment (start 133.2436 106.1664) (end 133.2436 106.9464) (width 0.25) (layer "F.Cu") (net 6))
 (segment (start 126.5986 99.7114) (end 126.5986 105.9714) (width 0.25) (layer "B.Cu") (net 7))
 (segment (start 127.9636 98.3464) (end 126.5986 99.7114) (width 0.25) (layer "B.Cu") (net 7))
 (segment (start 126.5986 105.9714) (end 125.6236 106.9464) (width 0.25) (layer "B.Cu") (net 7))
 (segment (start 128.1936 103.6564) (end 128.1936 103.9664) (width 0.25) (layer "F.Cu") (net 8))
 (segment (start 125.4236 100.8864) (end 128.1936 103.6564) (width 0.25) (layer "F.Cu") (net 8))
 (segment (start 128.1936 103.9664) (end 128.1636 103.9964) (width 0.25) (layer "F.Cu") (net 8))
 (segment (start 128.1636 103.9964) (end 128.1636 106.9464) (width 0.25) (layer "F.Cu") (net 8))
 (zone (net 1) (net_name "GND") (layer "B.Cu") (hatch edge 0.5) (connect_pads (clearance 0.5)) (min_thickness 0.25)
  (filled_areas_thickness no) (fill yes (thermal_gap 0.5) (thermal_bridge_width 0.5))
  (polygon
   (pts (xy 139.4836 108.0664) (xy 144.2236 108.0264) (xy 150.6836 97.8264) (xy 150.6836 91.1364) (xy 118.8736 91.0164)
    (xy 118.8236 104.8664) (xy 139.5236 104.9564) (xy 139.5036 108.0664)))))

